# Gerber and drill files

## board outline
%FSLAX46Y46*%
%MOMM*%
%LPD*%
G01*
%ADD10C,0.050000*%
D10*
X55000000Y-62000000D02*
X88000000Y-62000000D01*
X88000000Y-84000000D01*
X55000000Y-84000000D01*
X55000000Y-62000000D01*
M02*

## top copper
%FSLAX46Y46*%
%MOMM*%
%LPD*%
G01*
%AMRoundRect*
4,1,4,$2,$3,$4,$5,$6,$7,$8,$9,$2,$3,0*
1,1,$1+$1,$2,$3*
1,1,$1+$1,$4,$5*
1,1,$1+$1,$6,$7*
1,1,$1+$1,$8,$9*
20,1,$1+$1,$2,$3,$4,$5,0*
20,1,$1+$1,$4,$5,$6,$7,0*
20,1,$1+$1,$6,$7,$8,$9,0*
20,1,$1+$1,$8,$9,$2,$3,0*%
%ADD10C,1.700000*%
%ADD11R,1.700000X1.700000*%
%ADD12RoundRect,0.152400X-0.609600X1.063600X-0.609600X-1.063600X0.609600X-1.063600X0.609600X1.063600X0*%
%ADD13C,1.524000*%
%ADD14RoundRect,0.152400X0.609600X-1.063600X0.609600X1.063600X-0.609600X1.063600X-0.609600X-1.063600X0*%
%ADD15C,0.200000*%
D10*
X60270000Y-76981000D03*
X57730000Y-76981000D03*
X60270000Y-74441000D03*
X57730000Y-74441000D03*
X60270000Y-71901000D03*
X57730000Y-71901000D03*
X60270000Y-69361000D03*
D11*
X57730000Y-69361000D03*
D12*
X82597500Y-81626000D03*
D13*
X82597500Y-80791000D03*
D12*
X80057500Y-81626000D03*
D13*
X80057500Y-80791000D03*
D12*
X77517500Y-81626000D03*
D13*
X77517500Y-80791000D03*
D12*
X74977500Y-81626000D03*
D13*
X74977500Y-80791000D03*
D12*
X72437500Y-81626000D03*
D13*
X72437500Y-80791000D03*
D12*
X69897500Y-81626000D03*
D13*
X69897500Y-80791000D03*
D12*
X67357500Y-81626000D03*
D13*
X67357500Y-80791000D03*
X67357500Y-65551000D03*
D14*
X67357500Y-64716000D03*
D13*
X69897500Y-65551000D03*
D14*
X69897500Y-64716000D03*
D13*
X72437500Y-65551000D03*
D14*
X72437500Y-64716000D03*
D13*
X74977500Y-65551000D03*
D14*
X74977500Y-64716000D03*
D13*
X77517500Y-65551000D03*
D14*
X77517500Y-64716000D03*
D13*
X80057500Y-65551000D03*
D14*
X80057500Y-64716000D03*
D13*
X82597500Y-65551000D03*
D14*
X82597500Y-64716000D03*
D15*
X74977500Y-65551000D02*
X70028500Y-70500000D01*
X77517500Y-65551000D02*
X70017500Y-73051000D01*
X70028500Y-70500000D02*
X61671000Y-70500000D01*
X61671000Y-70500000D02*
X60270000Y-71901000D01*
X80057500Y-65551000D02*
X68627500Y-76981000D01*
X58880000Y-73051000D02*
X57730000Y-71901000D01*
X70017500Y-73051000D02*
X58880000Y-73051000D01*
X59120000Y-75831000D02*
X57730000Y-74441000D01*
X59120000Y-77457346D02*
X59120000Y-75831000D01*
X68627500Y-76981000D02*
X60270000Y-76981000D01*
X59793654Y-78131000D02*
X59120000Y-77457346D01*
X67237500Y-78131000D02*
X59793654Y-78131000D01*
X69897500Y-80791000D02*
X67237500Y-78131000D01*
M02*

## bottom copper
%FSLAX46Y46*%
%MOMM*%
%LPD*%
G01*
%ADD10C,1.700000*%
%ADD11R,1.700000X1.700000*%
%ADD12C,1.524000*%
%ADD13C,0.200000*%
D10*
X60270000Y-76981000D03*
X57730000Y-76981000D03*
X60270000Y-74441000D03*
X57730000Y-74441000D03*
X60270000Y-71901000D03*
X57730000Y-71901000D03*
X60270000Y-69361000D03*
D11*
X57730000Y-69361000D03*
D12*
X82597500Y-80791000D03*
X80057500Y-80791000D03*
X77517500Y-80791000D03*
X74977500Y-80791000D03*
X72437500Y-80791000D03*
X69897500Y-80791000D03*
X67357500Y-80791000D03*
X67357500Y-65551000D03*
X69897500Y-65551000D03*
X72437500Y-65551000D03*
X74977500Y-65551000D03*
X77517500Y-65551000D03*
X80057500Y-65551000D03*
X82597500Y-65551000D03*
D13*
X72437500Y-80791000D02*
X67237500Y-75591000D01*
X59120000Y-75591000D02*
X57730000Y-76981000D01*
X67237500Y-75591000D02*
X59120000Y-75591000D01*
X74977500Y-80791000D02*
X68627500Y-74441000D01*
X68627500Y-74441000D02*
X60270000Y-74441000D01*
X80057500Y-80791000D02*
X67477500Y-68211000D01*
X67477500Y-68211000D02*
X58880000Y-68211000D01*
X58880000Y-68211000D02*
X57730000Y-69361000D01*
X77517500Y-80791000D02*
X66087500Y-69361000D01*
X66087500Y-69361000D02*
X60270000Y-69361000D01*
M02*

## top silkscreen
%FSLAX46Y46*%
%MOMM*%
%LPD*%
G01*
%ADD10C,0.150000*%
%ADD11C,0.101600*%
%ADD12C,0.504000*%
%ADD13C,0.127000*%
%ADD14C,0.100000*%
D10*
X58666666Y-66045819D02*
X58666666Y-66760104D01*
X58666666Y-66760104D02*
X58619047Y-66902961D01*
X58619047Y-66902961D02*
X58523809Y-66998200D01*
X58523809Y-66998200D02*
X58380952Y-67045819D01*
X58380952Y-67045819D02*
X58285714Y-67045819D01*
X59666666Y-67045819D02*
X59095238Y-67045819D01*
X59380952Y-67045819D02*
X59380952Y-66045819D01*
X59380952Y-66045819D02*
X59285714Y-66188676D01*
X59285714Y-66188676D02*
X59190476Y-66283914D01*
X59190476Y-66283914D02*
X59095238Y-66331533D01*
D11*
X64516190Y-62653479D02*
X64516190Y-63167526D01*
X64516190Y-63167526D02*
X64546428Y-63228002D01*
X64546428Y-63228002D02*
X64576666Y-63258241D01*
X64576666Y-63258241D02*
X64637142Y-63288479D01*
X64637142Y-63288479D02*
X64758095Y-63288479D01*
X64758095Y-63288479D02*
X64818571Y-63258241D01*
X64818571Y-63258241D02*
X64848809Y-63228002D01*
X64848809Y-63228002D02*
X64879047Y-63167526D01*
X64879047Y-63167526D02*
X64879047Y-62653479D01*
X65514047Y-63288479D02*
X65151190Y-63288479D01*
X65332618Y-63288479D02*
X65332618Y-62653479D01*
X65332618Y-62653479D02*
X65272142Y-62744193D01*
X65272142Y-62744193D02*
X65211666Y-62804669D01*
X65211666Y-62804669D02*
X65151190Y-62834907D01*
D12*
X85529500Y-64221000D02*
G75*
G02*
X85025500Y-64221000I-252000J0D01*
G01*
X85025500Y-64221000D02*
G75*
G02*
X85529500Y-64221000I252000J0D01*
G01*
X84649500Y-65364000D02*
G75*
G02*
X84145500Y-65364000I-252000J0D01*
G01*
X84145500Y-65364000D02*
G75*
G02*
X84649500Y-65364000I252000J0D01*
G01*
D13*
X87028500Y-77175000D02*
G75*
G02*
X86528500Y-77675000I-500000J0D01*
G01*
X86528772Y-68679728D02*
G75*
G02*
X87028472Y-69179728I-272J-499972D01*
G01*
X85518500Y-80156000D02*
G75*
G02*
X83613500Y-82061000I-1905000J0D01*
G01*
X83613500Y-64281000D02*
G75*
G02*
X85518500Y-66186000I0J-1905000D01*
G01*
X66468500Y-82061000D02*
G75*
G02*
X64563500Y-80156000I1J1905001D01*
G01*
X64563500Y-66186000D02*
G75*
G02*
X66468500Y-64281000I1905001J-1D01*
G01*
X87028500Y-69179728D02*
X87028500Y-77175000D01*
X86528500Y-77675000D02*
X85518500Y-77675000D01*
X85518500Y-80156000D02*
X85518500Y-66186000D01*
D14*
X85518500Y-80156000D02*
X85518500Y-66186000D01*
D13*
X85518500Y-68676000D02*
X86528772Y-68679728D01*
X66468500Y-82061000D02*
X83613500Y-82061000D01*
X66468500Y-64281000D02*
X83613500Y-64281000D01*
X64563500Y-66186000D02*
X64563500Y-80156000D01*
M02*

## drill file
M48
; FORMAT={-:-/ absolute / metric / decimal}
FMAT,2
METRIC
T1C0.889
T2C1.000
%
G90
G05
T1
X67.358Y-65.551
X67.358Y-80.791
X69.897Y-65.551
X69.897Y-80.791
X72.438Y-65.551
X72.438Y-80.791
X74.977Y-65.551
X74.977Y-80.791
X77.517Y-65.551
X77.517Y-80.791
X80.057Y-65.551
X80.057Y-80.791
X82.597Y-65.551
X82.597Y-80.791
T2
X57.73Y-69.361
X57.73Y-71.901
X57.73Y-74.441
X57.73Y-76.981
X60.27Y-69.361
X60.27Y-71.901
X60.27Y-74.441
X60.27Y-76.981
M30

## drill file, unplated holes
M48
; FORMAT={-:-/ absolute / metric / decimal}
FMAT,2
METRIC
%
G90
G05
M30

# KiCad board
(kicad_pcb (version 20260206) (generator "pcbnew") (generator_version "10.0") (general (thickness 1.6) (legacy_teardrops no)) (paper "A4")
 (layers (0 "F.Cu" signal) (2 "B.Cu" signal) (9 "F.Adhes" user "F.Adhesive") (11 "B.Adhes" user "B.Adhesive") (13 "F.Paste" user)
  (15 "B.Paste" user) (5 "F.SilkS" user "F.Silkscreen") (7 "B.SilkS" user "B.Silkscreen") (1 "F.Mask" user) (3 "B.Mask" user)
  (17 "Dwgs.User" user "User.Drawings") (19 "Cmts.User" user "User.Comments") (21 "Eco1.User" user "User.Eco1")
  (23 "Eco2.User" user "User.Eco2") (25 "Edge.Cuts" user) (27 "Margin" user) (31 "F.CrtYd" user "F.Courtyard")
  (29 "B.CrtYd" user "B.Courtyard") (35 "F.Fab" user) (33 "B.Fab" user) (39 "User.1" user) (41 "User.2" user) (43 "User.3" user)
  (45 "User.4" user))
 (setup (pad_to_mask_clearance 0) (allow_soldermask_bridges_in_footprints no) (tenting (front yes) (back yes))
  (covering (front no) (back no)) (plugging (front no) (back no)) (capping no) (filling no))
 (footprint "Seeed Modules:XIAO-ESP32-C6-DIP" (layer "F.Cu") (at 74.9775 73.171)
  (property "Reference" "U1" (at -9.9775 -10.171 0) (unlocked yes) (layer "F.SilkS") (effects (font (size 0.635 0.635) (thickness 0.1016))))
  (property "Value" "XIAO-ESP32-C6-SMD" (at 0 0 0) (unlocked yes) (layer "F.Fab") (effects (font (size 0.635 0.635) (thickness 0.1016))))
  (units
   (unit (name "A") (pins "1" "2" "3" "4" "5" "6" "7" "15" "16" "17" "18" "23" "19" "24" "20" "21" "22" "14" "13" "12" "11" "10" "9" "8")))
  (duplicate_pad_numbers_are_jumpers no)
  (fp_line (start -10.414 -6.985) (end -10.414 6.985) (stroke (width 0.127) (type solid)) (layer "F.SilkS"))
  (fp_line (start -8.509 -8.89) (end 8.636 -8.89) (stroke (width 0.127) (type solid)) (layer "F.SilkS"))
  (fp_line (start -8.509 8.89) (end 8.636 8.89) (stroke (width 0.127) (type solid)) (layer "F.SilkS"))
  (fp_line (start 10.541 -4.495) (end 11.551272 -4.491272) (stroke (width 0.127) (type solid)) (layer "F.SilkS"))
  (fp_line (start 10.541 6.985) (end 10.541 -6.985) (stroke (width 0.1) (type solid)) (layer "F.SilkS"))
  (fp_line (start 10.541 6.985) (end 10.541 -6.985) (stroke (width 0.127) (type solid)) (layer "F.SilkS"))
  (fp_line (start 11.551 4.504) (end 10.541 4.504) (stroke (width 0.127) (type solid)) (layer "F.SilkS"))
  (fp_line (start 12.051 -3.991272) (end 12.051 4.004) (stroke (width 0.127) (type solid)) (layer "F.SilkS"))
  (fp_arc (start -10.414 -6.985) (mid -9.856038 -8.332038) (end -8.509 -8.89) (stroke (width 0.127) (type solid)) (layer "F.SilkS"))
  (fp_arc (start -8.509 8.89) (mid -9.856038 8.332038) (end -10.414 6.985) (stroke (width 0.127) (type solid)) (layer "F.SilkS"))
  (fp_arc (start 8.636 -8.89) (mid 9.983038 -8.332038) (end 10.541 -6.985) (stroke (width 0.127) (type solid)) (layer "F.SilkS"))
  (fp_arc (start 10.541 6.985) (mid 9.983038 8.332038) (end 8.636 8.89) (stroke (width 0.127) (type solid)) (layer "F.SilkS"))
  (fp_arc (start 11.551272 -4.491272) (mid 11.904644 -4.344724) (end 12.051 -3.991272) (stroke (width 0.127) (type default))
   (layer "F.SilkS"))
  (fp_arc (start 12.051 4.004) (mid 11.904553 4.357553) (end 11.551 4.504) (stroke (width 0.127) (type default)) (layer "F.SilkS"))
  (fp_circle (center 9.42 -7.807) (end 9.674 -7.807) (stroke (width 0.5) (type solid)) (fill yes) (layer "F.SilkS"))
  (fp_circle (center 10.3 -8.95) (end 10.554 -8.95) (stroke (width 0.5) (type solid)) (fill yes) (layer "F.SilkS"))
  (pad "1" smd roundrect (at 7.62 -8.455 90) (size 2.432 1.524) (layers "F.Cu" "F.Mask") (roundrect_rratio 0.1)
   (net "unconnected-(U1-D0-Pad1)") (thermal_bridge_angle 45))
  (pad "1" thru_hole circle (at 7.62 -7.62 90) (size 1.524 1.524) (drill 0.889) (layers "*.Cu" "*.Mask") (remove_unused_layers no)
   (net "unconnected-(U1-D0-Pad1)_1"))
  (pad "2" smd roundrect (at 5.08 -8.455 90) (size 2.432 1.524) (layers "F.Cu" "F.Mask") (roundrect_rratio 0.1) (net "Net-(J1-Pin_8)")
   (thermal_bridge_angle 45))
  (pad "2" thru_hole circle (at 5.08 -7.62 90) (size 1.524 1.524) (drill 0.889) (layers "*.Cu" "*.Mask") (remove_unused_layers no)
   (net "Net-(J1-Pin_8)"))
  (pad "3" smd roundrect (at 2.54 -8.455 90) (size 2.432 1.524) (layers "F.Cu" "F.Mask") (roundrect_rratio 0.1) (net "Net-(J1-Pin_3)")
   (thermal_bridge_angle 45))
  (pad "3" thru_hole circle (at 2.54 -7.62 90) (size 1.524 1.524) (drill 0.889) (layers "*.Cu" "*.Mask") (remove_unused_layers no)
   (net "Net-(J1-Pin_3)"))
  (pad "4" smd roundrect (at 0 -8.455 90) (size 2.432 1.524) (layers "F.Cu" "F.Mask") (roundrect_rratio 0.1) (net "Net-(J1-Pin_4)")
   (thermal_bridge_angle 45))
  (pad "4" thru_hole circle (at 0 -7.62 90) (size 1.524 1.524) (drill 0.889) (layers "*.Cu" "*.Mask") (remove_unused_layers no)
   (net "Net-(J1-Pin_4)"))
  (pad "5" smd roundrect (at -2.54 -8.455 90) (size 2.432 1.524) (layers "F.Cu" "F.Mask") (roundrect_rratio 0.1)
   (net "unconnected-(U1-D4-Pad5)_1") (thermal_bridge_angle 45))
  (pad "5" thru_hole circle (at -2.54 -7.62 90) (size 1.524 1.524) (drill 0.889) (layers "*.Cu" "*.Mask") (remove_unused_layers no)
   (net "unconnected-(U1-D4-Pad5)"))
  (pad "6" smd roundrect (at -5.08 -8.455 90) (size 2.432 1.524) (layers "F.Cu" "F.Mask") (roundrect_rratio 0.1)
   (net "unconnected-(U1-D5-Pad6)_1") (thermal_bridge_angle 45))
  (pad "6" thru_hole circle (at -5.08 -7.62 90) (size 1.524 1.524) (drill 0.889) (layers "*.Cu" "*.Mask") (remove_unused_layers no)
   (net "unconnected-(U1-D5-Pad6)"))
  (pad "7" smd roundrect (at -7.62 -8.455 90) (size 2.432 1.524) (layers "F.Cu" "F.Mask") (roundrect_rratio 0.1)
   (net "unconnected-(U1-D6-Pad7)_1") (thermal_bridge_angle 45))
  (pad "7" thru_hole circle (at -7.62 -7.62 90) (size 1.524 1.524) (drill 0.889) (layers "*.Cu" "*.Mask") (remove_unused_layers no)
   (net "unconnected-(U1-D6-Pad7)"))
  (pad "8" thru_hole circle (at -7.62 7.62 270) (size 1.524 1.524) (drill 0.889) (layers "*.Cu" "*.Mask") (remove_unused_layers no)
   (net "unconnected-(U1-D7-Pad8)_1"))
  (pad "8" smd roundrect (at -7.62 8.455 270) (size 2.432 1.524) (layers "F.Cu" "F.Mask") (roundrect_rratio 0.1)
   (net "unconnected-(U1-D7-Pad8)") (thermal_bridge_angle 45))
  (pad "9" thru_hole circle (at -5.08 7.62 270) (size 1.524 1.524) (drill 0.889) (layers "*.Cu" "*.Mask") (remove_unused_layers no)
   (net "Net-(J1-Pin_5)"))
  (pad "9" smd roundrect (at -5.08 8.455 270) (size 2.432 1.524) (layers "F.Cu" "F.Mask") (roundrect_rratio 0.1) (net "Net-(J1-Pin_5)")
   (thermal_bridge_angle 45))
  (pad "10" thru_hole circle (at -2.54 7.62 270) (size 1.524 1.524) (drill 0.889) (layers "*.Cu" "*.Mask") (remove_unused_layers no)
   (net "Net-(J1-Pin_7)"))
  (pad "10" smd roundrect (at -2.54 8.455 270) (size 2.432 1.524) (layers "F.Cu" "F.Mask") (roundrect_rratio 0.1) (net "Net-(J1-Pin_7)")
   (thermal_bridge_angle 45))
  (pad "11" thru_hole circle (at 0 7.62 270) (size 1.524 1.524) (drill 0.889) (layers "*.Cu" "*.Mask") (remove_unused_layers no)
   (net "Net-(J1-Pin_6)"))
  (pad "11" smd roundrect (at 0 8.455 270) (size 2.432 1.524) (layers "F.Cu" "F.Mask") (roundrect_rratio 0.1) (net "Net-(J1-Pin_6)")
   (thermal_bridge_angle 45))
  (pad "12" thru_hole circle (at 2.54 7.62 270) (size 1.524 1.524) (drill 0.889) (layers "*.Cu" "*.Mask") (remove_unused_layers no)
   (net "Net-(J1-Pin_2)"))
  (pad "12" smd roundrect (at 2.54 8.455 270) (size 2.432 1.524) (layers "F.Cu" "F.Mask") (roundrect_rratio 0.1) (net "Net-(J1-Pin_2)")
   (thermal_bridge_angle 45))
  (pad "13" thru_hole circle (at 5.08 7.62 270) (size 1.524 1.524) (drill 0.889) (layers "*.Cu" "*.Mask") (remove_unused_layers no)
   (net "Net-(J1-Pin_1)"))
  (pad "13" smd roundrect (at 5.08 8.455 270) (size 2.432 1.524) (layers "F.Cu" "F.Mask") (roundrect_rratio 0.1) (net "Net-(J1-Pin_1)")
   (thermal_bridge_angle 45))
  (pad "14" thru_hole circle (at 7.62 7.62 270) (size 1.524 1.524) (drill 0.889) (layers "*.Cu" "*.Mask") (remove_unused_layers no)
   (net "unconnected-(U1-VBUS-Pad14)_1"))
  (pad "14" smd roundrect (at 7.62 8.455 270) (size 2.432 1.524) (layers "F.Cu" "F.Mask") (roundrect_rratio 0.1)
   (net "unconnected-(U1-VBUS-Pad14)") (thermal_bridge_angle 45)))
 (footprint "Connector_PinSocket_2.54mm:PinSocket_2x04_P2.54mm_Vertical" (layer "B.Cu") (at 57.73 69.361 180)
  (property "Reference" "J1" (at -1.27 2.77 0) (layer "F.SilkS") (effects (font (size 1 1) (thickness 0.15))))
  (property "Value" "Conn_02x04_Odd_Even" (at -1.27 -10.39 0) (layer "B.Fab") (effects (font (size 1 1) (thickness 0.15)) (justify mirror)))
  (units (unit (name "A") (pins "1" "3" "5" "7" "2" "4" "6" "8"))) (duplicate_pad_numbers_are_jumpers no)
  (pad "1" thru_hole rect (at 0 0 180) (size 1.7 1.7) (drill 1) (layers "*.Cu" "*.Mask") (remove_unused_layers no) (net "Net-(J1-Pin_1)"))
  (pad "2" thru_hole circle (at -2.54 0 180) (size 1.7 1.7) (drill 1) (layers "*.Cu" "*.Mask") (remove_unused_layers no)
   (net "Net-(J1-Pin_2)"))
  (pad "3" thru_hole circle (at 0 -2.54 180) (size 1.7 1.7) (drill 1) (layers "*.Cu" "*.Mask") (remove_unused_layers no)
   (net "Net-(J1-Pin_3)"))
  (pad "4" thru_hole circle (at -2.54 -2.54 180) (size 1.7 1.7) (drill 1) (layers "*.Cu" "*.Mask") (remove_unused_layers no)
   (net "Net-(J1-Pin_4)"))
  (pad "5" thru_hole circle (at 0 -5.08 180) (size 1.7 1.7) (drill 1) (layers "*.Cu" "*.Mask") (remove_unused_layers no)
   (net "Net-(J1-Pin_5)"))
  (pad "6" thru_hole circle (at -2.54 -5.08 180) (size 1.7 1.7) (drill 1) (layers "*.Cu" "*.Mask") (remove_unused_layers no)
   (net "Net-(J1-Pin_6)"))
  (pad "7" thru_hole circle (at 0 -7.62 180) (size 1.7 1.7) (drill 1) (layers "*.Cu" "*.Mask") (remove_unused_layers no)
   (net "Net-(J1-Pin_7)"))
  (pad "8" thru_hole circle (at -2.54 -7.62 180) (size 1.7 1.7) (drill 1) (layers "*.Cu" "*.Mask") (remove_unused_layers no)
   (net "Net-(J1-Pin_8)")))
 (gr_rect (start 55 62) (end 88 84) (stroke (width 0.05) (type default)) (fill no) (layer "Edge.Cuts"))
 (segment (start 67.2375 75.591) (end 59.12 75.591) (width 0.2) (layer "B.Cu") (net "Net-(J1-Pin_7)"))
 (segment (start 59.12 75.591) (end 57.73 76.981) (width 0.2) (layer "B.Cu") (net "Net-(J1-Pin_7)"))
 (segment (start 72.4375 80.791) (end 67.2375 75.591) (width 0.2) (layer "B.Cu") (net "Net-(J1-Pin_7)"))
 (segment (start 59.12 77.457346) (end 59.12 75.831) (width 0.2) (layer "F.Cu") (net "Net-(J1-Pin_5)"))
 (segment (start 67.2375 78.131) (end 59.793654 78.131) (width 0.2) (layer "F.Cu") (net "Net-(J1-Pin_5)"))
 (segment (start 59.793654 78.131) (end 59.12 77.457346) (width 0.2) (layer "F.Cu") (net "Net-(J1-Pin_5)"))
 (segment (start 69.8975 80.791) (end 67.2375 78.131) (width 0.2) (layer "F.Cu") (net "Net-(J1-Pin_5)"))
 (segment (start 59.12 75.831) (end 57.73 74.441) (width 0.2) (layer "F.Cu") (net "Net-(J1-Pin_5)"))
 (segment (start 70.0175 73.051) (end 58.88 73.051) (width 0.2) (layer "F.Cu") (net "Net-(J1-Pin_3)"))
 (segment (start 77.5175 65.551) (end 70.0175 73.051) (width 0.2) (layer "F.Cu") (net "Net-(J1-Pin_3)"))
 (segment (start 58.88 73.051) (end 57.73 71.901) (width 0.2) (layer "F.Cu") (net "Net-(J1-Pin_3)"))
 (segment (start 70.0285 70.5) (end 61.671 70.5) (width 0.2) (layer "F.Cu") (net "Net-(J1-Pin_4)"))
 (segment (start 61.671 70.5) (end 60.27 71.901) (width 0.2) (layer "F.Cu") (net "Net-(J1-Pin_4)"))
 (segment (start 74.9775 65.551) (end 70.0285 70.5) (width 0.2) (layer "F.Cu") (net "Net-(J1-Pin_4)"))
 (segment (start 68.6275 76.981) (end 60.27 76.981) (width 0.2) (layer "F.Cu") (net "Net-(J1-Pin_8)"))
 (segment (start 80.0575 65.551) (end 68.6275 76.981) (width 0.2) (layer "F.Cu") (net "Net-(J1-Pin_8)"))
 (segment (start 77.5175 80.791) (end 66.0875 69.361) (width 0.2) (layer "B.Cu") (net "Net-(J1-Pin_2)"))
 (segment (start 66.0875 69.361) (end 60.27 69.361) (width 0.2) (layer "B.Cu") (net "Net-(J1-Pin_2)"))
 (segment (start 68.6275 74.441) (end 60.27 74.441) (width 0.2) (layer "B.Cu") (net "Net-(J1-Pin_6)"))
 (segment (start 74.9775 80.791) (end 68.6275 74.441) (width 0.2) (layer "B.Cu") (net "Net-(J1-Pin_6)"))
 (segment (start 67.4775 68.211) (end 58.88 68.211) (width 0.2) (layer "B.Cu") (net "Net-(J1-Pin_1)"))
 (segment (start 80.0575 80.791) (end 67.4775 68.211) (width 0.2) (layer "B.Cu") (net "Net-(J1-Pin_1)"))
 (segment (start 58.88 68.211) (end 57.73 69.361) (width 0.2) (layer "B.Cu") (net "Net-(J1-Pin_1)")))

